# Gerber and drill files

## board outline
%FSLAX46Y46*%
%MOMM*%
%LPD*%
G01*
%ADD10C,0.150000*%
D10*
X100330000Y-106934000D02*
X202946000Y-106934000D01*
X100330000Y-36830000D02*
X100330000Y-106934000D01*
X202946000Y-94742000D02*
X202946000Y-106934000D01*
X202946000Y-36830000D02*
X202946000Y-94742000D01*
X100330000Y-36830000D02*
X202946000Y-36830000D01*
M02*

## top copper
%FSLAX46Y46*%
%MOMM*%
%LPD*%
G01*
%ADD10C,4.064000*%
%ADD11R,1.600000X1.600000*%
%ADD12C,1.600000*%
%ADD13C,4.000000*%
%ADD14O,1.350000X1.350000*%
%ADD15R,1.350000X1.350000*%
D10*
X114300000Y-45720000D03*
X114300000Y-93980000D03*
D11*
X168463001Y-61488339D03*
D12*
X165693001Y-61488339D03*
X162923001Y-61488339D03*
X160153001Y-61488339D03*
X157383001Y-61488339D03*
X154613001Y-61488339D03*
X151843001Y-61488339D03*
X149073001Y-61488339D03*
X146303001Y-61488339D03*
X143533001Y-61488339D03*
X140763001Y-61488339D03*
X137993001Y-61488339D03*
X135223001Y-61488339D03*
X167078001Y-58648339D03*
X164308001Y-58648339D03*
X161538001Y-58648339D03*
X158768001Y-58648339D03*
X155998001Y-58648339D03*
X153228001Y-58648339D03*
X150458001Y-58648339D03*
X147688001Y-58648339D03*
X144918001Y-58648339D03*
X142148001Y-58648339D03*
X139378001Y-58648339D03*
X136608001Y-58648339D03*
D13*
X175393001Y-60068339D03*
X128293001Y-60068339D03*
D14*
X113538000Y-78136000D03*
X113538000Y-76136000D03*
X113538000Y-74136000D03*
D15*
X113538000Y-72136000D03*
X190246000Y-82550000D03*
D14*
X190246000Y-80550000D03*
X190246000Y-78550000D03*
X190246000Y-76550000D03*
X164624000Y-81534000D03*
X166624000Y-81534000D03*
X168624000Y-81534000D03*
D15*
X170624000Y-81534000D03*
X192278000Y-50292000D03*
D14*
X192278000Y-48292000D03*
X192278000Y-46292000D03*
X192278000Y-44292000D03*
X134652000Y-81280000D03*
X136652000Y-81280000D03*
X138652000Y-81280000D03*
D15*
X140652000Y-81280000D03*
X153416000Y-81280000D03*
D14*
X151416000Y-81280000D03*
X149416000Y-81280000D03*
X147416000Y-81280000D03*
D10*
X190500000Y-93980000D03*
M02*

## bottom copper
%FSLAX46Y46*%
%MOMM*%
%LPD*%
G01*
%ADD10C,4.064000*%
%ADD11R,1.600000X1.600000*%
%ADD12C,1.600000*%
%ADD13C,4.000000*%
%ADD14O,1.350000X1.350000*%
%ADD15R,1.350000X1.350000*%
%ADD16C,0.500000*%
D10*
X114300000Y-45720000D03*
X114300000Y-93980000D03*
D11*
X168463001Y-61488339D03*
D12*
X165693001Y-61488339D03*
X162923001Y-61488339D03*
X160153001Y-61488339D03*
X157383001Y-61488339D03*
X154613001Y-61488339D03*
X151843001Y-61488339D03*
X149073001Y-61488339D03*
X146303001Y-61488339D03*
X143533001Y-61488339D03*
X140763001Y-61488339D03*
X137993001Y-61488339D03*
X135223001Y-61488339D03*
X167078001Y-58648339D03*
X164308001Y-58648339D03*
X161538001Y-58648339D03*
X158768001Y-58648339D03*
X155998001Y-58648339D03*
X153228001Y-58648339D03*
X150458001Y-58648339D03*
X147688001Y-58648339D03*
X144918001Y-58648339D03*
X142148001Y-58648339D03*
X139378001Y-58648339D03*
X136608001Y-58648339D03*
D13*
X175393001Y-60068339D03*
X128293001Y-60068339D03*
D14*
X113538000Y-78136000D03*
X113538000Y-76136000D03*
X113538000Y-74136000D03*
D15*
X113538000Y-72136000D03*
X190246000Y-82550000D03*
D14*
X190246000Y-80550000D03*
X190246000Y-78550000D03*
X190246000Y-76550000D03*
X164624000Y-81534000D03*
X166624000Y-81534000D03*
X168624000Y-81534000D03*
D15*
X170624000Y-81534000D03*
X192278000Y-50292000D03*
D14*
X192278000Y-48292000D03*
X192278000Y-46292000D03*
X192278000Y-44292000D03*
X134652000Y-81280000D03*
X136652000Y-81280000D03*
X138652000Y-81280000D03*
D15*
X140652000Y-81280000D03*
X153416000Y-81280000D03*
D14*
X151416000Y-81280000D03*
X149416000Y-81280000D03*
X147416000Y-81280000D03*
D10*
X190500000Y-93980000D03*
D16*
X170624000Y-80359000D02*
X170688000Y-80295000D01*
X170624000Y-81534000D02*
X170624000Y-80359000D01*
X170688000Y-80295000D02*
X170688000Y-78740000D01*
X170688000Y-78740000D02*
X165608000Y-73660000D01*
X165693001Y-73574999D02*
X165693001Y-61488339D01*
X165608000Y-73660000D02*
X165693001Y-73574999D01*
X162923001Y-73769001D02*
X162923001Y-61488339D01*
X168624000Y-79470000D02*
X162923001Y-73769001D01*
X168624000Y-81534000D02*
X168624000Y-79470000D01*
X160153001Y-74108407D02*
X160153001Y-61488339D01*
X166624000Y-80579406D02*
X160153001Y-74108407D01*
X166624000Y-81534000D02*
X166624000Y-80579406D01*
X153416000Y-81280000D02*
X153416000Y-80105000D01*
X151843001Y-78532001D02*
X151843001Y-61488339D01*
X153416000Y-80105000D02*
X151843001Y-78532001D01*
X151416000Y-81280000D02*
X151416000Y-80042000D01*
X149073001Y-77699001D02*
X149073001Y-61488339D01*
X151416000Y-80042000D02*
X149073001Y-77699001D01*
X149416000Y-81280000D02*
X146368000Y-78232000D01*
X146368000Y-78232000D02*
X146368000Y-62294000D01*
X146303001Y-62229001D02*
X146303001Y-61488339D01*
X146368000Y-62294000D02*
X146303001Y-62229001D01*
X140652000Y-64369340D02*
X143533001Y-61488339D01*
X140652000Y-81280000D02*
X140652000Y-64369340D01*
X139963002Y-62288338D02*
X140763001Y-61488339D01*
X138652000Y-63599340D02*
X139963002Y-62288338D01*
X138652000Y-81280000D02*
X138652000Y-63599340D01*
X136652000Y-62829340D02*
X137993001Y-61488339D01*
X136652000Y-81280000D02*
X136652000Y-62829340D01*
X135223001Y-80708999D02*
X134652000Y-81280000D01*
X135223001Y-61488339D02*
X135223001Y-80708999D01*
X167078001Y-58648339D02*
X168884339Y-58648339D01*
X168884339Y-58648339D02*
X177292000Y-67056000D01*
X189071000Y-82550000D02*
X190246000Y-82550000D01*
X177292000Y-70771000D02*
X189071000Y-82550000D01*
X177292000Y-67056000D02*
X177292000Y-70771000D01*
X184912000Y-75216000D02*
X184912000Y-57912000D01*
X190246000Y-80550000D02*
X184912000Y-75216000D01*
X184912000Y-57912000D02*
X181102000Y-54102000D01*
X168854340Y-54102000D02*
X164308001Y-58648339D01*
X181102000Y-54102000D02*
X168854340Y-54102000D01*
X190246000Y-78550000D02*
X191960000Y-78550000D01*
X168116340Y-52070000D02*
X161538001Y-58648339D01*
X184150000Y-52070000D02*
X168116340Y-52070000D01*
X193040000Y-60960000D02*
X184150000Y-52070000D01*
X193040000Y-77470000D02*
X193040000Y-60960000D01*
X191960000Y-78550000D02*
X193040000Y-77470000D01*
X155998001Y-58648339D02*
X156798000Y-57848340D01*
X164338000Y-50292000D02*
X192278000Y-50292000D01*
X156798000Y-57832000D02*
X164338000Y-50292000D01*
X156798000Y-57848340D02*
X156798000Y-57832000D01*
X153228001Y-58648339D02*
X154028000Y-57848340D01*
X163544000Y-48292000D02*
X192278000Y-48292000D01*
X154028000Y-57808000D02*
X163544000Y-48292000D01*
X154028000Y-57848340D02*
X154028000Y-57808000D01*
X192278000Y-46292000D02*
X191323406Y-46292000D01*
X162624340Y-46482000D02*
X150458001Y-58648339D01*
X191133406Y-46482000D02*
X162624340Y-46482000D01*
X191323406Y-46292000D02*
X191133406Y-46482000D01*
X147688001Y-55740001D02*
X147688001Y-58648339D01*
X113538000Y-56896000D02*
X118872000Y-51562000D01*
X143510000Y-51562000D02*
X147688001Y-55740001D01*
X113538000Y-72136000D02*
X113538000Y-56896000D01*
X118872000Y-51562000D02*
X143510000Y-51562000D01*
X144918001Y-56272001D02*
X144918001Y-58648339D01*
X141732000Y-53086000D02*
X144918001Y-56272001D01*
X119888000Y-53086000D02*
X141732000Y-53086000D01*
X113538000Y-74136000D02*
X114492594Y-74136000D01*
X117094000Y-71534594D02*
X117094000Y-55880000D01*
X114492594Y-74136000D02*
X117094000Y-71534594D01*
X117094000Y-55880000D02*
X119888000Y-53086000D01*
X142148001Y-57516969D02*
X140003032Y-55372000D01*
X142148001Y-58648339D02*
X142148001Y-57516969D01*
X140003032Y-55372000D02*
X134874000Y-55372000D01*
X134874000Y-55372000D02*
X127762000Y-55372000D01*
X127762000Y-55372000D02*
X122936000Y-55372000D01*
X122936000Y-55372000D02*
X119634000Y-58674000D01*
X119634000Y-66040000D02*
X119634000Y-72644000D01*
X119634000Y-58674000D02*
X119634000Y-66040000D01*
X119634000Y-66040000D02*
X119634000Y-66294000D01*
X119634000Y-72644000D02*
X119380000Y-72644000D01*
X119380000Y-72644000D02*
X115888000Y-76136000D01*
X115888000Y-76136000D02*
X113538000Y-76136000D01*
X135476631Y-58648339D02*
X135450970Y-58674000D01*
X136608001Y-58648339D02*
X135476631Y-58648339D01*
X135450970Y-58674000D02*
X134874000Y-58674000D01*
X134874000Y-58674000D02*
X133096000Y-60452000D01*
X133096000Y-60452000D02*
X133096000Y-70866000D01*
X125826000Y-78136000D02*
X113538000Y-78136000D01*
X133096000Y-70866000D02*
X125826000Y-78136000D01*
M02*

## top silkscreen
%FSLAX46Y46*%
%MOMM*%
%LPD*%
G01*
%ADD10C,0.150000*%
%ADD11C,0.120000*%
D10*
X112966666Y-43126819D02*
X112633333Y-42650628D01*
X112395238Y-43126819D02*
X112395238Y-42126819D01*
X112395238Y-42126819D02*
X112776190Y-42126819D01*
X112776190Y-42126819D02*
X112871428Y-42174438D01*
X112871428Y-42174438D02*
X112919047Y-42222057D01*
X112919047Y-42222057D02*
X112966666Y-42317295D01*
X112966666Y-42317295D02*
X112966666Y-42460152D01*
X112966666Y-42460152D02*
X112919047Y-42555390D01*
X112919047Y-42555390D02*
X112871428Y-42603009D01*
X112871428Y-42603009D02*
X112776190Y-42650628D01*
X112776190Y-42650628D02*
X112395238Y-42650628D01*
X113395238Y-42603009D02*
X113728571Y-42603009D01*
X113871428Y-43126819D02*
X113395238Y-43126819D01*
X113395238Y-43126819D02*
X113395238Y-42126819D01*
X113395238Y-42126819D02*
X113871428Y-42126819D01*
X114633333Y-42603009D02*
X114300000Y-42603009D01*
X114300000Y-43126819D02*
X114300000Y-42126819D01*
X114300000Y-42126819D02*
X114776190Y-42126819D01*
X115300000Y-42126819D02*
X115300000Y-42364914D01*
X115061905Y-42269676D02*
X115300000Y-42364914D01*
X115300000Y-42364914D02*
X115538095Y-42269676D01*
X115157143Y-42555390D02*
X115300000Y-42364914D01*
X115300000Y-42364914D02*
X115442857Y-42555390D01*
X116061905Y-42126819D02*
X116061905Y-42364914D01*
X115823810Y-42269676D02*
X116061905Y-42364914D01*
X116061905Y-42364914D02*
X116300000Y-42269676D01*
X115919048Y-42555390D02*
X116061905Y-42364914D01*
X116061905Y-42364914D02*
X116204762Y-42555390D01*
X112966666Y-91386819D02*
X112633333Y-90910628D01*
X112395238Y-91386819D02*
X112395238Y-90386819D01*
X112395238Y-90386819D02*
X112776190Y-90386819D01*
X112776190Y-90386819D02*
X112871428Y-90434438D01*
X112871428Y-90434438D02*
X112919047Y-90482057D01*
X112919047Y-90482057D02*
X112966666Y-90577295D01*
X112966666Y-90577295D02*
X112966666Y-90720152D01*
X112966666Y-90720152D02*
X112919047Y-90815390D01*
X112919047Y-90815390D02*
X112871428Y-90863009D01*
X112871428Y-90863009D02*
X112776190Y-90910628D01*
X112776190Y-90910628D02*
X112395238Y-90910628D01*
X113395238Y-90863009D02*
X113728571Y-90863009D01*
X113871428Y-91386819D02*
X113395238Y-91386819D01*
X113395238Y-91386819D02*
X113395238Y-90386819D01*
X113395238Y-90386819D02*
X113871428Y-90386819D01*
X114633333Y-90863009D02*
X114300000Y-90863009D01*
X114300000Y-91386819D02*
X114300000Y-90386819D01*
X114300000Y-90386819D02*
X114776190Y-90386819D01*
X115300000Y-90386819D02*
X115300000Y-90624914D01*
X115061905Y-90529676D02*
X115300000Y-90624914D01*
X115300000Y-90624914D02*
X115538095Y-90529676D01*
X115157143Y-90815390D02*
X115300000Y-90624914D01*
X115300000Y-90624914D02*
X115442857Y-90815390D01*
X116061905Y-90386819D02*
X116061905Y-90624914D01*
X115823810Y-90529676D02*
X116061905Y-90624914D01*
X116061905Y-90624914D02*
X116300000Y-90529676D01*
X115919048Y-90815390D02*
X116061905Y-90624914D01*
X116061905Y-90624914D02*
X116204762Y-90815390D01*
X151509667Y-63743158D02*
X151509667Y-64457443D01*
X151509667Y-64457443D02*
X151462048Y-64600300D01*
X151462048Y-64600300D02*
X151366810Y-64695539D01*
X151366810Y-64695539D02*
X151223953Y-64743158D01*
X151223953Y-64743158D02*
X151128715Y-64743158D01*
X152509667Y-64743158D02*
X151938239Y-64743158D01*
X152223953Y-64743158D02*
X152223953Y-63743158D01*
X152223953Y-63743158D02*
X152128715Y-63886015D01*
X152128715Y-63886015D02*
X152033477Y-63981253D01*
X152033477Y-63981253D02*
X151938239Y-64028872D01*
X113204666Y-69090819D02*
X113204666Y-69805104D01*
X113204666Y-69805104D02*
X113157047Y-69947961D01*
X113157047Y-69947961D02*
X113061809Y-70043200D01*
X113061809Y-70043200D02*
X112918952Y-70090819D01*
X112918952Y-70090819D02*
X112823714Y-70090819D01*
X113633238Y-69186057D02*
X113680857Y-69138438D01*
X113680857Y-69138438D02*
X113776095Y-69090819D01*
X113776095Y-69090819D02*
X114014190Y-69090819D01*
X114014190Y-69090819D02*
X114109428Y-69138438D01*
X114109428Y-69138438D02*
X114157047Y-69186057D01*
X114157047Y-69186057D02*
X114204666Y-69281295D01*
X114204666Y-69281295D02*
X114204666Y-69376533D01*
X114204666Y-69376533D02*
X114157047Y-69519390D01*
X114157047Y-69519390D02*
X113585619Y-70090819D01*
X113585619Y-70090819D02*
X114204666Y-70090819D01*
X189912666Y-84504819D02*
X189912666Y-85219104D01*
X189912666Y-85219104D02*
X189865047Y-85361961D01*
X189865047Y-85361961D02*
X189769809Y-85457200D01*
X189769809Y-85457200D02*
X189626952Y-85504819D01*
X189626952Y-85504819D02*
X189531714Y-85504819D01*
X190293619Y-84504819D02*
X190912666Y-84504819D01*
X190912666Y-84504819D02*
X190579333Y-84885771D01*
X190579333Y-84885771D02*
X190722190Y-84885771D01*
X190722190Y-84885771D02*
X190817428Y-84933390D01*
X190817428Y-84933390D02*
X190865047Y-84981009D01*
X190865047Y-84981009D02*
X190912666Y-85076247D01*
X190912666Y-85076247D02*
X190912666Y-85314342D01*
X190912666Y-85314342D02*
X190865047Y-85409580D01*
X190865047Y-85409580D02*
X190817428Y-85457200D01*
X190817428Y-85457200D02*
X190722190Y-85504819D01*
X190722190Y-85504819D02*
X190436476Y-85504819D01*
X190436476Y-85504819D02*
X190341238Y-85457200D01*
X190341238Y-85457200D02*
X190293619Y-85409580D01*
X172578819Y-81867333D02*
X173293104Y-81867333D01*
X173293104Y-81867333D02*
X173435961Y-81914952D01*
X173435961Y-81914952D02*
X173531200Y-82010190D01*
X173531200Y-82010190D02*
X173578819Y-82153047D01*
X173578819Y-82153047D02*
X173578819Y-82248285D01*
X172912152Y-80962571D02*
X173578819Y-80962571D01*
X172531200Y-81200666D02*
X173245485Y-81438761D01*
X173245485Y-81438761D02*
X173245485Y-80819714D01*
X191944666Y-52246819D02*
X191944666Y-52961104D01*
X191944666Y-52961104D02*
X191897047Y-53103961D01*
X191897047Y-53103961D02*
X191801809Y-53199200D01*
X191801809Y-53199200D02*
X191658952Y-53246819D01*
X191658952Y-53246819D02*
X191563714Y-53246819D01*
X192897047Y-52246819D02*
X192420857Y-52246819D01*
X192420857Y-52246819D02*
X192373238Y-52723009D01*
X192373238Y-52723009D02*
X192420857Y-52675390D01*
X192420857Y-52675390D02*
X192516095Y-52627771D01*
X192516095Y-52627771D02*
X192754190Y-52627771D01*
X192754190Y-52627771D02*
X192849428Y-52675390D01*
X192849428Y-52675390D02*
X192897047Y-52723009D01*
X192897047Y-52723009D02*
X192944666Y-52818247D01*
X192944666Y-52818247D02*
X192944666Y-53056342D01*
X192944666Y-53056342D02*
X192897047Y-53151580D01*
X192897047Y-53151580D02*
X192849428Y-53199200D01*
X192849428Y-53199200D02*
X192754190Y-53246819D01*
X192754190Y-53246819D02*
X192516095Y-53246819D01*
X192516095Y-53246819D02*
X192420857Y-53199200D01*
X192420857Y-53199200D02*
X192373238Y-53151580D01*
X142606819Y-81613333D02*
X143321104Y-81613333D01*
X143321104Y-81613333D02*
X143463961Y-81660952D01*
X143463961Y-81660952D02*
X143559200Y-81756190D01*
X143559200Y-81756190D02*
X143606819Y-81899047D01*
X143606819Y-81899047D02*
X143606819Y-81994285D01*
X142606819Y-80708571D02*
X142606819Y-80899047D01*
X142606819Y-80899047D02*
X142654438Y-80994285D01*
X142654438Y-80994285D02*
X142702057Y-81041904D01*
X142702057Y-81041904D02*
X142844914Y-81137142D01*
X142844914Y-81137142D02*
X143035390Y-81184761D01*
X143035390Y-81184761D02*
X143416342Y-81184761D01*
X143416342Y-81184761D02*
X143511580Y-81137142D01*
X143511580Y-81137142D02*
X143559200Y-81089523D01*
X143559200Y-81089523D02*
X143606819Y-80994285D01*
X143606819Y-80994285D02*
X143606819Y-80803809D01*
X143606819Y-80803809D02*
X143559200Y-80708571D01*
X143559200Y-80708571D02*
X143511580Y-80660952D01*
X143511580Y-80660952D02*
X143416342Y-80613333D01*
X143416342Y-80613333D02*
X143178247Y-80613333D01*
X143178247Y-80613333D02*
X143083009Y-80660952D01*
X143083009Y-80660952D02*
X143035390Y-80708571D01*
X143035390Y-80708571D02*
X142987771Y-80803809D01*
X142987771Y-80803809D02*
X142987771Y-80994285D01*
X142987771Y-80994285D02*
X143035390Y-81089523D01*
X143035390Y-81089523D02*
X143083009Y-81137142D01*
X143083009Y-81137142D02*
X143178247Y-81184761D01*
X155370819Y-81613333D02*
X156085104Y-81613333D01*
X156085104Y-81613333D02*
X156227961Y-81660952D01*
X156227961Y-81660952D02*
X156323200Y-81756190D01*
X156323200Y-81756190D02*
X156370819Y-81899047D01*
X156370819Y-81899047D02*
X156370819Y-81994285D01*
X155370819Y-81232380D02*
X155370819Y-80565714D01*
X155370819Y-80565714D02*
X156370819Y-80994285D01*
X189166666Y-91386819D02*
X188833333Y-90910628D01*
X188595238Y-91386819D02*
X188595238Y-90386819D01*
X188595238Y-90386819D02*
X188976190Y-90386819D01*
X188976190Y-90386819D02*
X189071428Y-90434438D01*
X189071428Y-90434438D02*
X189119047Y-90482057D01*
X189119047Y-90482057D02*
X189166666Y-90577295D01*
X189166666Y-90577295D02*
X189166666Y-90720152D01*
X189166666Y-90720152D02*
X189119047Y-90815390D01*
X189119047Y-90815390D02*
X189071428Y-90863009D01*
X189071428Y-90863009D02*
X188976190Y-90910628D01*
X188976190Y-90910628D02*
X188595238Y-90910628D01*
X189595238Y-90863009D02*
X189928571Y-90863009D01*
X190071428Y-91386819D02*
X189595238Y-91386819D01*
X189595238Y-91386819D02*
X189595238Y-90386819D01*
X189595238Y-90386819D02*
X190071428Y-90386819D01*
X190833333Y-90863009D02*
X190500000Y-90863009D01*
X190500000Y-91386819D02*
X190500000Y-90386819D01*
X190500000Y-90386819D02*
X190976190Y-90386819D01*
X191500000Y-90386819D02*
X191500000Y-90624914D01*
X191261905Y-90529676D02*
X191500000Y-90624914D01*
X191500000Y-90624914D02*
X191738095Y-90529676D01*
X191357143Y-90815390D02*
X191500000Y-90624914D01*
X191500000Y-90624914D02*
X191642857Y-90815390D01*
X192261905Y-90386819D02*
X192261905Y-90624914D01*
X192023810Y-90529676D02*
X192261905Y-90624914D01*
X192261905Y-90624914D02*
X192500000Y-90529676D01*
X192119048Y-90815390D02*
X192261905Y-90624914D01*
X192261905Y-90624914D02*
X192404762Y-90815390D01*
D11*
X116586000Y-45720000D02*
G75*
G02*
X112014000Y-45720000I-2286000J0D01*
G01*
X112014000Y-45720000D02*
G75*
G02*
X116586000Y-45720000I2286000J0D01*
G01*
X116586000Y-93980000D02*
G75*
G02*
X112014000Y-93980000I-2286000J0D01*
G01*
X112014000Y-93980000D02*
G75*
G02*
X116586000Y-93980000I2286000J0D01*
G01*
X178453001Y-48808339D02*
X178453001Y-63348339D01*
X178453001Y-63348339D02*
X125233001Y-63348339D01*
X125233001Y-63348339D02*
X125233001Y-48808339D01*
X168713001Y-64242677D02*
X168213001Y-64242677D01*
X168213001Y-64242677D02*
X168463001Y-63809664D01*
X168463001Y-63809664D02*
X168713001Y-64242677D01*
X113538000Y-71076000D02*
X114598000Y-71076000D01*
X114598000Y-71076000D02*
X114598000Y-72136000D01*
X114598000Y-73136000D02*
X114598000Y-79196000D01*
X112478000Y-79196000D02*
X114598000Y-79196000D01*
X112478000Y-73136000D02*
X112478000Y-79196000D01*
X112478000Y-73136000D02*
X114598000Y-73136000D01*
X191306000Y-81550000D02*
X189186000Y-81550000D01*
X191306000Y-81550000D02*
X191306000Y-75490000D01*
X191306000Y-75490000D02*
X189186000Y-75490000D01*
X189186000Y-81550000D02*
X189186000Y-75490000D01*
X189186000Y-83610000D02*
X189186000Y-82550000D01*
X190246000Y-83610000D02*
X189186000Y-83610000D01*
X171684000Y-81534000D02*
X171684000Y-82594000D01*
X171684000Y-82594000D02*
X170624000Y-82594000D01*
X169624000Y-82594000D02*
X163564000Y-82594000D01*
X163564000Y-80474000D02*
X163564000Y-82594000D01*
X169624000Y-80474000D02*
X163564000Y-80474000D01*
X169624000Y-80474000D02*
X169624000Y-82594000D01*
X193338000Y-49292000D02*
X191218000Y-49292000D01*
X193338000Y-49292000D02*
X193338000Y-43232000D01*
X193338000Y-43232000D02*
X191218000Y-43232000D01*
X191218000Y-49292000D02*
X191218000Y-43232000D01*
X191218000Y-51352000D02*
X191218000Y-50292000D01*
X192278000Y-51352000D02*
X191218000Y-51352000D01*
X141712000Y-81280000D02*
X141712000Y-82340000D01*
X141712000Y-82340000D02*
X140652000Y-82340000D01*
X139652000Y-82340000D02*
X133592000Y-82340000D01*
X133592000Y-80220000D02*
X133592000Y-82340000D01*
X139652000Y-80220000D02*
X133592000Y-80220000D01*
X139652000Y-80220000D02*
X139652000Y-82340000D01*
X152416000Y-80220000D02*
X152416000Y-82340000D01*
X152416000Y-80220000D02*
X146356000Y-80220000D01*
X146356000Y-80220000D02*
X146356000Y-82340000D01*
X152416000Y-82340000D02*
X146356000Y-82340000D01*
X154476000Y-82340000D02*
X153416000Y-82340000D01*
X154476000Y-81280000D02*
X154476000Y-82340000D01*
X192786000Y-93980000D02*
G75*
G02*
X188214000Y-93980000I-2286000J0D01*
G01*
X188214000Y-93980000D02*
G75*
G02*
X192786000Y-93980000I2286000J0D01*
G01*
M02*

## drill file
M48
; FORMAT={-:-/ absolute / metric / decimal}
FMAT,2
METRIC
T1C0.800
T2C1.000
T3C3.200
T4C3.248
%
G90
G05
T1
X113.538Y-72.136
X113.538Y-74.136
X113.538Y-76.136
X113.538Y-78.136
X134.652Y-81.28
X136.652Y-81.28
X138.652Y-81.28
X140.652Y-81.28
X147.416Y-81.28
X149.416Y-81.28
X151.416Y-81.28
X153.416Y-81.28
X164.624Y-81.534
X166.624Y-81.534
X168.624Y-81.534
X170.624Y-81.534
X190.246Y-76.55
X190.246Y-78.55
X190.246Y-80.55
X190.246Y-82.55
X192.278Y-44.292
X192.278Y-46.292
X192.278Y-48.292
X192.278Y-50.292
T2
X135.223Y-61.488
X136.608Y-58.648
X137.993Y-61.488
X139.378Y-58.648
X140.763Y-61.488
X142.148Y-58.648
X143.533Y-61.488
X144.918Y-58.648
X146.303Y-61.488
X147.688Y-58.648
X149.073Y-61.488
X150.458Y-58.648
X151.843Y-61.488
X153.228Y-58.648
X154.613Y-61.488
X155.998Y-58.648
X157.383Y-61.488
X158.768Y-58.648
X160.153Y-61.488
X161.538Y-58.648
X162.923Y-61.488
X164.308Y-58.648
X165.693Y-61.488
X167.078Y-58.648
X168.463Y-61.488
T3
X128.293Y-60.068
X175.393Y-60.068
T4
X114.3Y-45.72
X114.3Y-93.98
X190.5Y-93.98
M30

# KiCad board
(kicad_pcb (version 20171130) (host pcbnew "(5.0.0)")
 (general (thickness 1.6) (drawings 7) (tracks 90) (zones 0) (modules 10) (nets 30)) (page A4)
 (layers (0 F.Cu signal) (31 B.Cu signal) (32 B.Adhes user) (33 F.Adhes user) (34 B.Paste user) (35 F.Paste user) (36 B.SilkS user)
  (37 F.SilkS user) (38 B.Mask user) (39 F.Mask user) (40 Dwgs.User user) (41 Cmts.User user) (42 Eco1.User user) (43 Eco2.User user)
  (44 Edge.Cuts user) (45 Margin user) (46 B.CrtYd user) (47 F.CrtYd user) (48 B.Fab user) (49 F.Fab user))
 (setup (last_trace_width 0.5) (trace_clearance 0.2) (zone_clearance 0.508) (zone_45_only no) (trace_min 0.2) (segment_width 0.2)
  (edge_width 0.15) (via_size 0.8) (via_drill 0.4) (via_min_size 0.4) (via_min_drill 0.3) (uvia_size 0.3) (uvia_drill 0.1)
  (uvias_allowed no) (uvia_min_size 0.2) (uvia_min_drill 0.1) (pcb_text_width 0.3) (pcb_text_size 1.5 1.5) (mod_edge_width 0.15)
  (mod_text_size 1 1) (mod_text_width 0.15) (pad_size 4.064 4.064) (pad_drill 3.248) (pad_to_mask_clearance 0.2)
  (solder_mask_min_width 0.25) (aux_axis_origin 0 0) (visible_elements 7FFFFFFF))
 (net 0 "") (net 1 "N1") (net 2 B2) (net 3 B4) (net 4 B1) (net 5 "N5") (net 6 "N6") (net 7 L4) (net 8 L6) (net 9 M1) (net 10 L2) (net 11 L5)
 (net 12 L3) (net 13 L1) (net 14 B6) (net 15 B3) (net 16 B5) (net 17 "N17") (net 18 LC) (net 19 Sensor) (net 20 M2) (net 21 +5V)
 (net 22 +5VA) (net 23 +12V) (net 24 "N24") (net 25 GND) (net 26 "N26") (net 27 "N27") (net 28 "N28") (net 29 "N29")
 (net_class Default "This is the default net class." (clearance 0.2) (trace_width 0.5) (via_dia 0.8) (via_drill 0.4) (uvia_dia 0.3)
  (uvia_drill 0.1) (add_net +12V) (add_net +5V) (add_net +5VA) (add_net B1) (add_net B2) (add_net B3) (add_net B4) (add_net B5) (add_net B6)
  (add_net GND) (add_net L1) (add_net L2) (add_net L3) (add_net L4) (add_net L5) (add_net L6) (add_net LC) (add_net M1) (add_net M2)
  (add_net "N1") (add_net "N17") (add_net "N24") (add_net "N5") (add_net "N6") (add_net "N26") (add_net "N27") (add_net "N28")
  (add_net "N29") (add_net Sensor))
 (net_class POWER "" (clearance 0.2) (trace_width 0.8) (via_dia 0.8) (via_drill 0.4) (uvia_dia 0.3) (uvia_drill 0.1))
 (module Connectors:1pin (layer F.Cu) (at 114.3 45.72)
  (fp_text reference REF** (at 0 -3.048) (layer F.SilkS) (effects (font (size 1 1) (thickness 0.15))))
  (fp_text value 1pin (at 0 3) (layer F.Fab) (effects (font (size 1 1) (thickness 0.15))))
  (fp_circle (center 0 0) (end 0 -2.286) (layer F.SilkS) (width 0.12))
  (pad 1 thru_hole circle (at 0 0) (size 4.064 4.064) (drill 3.248) (layers *.Cu *.Mask)))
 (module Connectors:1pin (layer F.Cu) (at 114.3 93.98)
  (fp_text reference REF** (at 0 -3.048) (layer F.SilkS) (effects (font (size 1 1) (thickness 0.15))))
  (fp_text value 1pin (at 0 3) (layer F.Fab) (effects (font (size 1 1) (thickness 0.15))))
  (fp_circle (center 0 0) (end 0 -2.286) (layer F.SilkS) (width 0.12))
  (pad 1 thru_hole circle (at 0 0) (size 4.064 4.064) (drill 3.248) (layers *.Cu *.Mask)))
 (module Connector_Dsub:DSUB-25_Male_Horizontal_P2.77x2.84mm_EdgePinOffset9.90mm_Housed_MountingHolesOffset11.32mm (layer F.Cu)
  (at 168.463001 61.488339 180)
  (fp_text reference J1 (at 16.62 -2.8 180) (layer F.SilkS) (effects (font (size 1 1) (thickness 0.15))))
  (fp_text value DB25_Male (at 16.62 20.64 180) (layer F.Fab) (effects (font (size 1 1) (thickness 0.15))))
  (fp_line (start -9.99 12.68) (end -9.99 -1.86) (layer F.SilkS) (width 0.12))
  (fp_line (start -9.99 -1.86) (end 43.23 -1.86) (layer F.SilkS) (width 0.12))
  (fp_line (start 43.23 -1.86) (end 43.23 12.68) (layer F.SilkS) (width 0.12))
  (fp_line (start -0.25 -2.754338) (end 0.25 -2.754338) (layer F.SilkS) (width 0.12))
  (fp_line (start 0.25 -2.754338) (end 0 -2.321325) (layer F.SilkS) (width 0.12))
  (fp_line (start 0 -2.321325) (end -0.25 -2.754338) (layer F.SilkS) (width 0.12))
  (pad 1 thru_hole rect (at 0 0 180) (size 1.6 1.6) (drill 1) (layers *.Cu *.Mask) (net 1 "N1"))
  (pad 2 thru_hole circle (at 2.77 0 180) (size 1.6 1.6) (drill 1) (layers *.Cu *.Mask) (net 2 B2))
  (pad 3 thru_hole circle (at 5.54 0 180) (size 1.6 1.6) (drill 1) (layers *.Cu *.Mask) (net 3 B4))
  (pad 4 thru_hole circle (at 8.31 0 180) (size 1.6 1.6) (drill 1) (layers *.Cu *.Mask) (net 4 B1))
  (pad 5 thru_hole circle (at 11.08 0 180) (size 1.6 1.6) (drill 1) (layers *.Cu *.Mask) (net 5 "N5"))
  (pad 6 thru_hole circle (at 13.85 0 180) (size 1.6 1.6) (drill 1) (layers *.Cu *.Mask) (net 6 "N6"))
  (pad 7 thru_hole circle (at 16.62 0 180) (size 1.6 1.6) (drill 1) (layers *.Cu *.Mask) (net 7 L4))
  (pad 8 thru_hole circle (at 19.39 0 180) (size 1.6 1.6) (drill 1) (layers *.Cu *.Mask) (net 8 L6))
  (pad 9 thru_hole circle (at 22.16 0 180) (size 1.6 1.6) (drill 1) (layers *.Cu *.Mask) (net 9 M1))
  (pad 10 thru_hole circle (at 24.93 0 180) (size 1.6 1.6) (drill 1) (layers *.Cu *.Mask) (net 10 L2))
  (pad 11 thru_hole circle (at 27.7 0 180) (size 1.6 1.6) (drill 1) (layers *.Cu *.Mask) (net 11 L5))
  (pad 12 thru_hole circle (at 30.47 0 180) (size 1.6 1.6) (drill 1) (layers *.Cu *.Mask) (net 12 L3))
  (pad 13 thru_hole circle (at 33.24 0 180) (size 1.6 1.6) (drill 1) (layers *.Cu *.Mask) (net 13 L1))
  (pad 14 thru_hole circle (at 1.385 2.84 180) (size 1.6 1.6) (drill 1) (layers *.Cu *.Mask) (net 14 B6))
  (pad 15 thru_hole circle (at 4.155 2.84 180) (size 1.6 1.6) (drill 1) (layers *.Cu *.Mask) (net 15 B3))
  (pad 16 thru_hole circle (at 6.925 2.84 180) (size 1.6 1.6) (drill 1) (layers *.Cu *.Mask) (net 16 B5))
  (pad 17 thru_hole circle (at 9.695 2.84 180) (size 1.6 1.6) (drill 1) (layers *.Cu *.Mask) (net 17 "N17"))
  (pad 18 thru_hole circle (at 12.465 2.84 180) (size 1.6 1.6) (drill 1) (layers *.Cu *.Mask) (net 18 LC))
  (pad 19 thru_hole circle (at 15.235 2.84 180) (size 1.6 1.6) (drill 1) (layers *.Cu *.Mask) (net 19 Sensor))
  (pad 20 thru_hole circle (at 18.005 2.84 180) (size 1.6 1.6) (drill 1) (layers *.Cu *.Mask) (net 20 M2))
  (pad 21 thru_hole circle (at 20.775 2.84 180) (size 1.6 1.6) (drill 1) (layers *.Cu *.Mask) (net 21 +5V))
  (pad 22 thru_hole circle (at 23.545 2.84 180) (size 1.6 1.6) (drill 1) (layers *.Cu *.Mask) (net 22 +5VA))
  (pad 23 thru_hole circle (at 26.315 2.84 180) (size 1.6 1.6) (drill 1) (layers *.Cu *.Mask) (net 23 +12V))
  (pad 24 thru_hole circle (at 29.085 2.84 180) (size 1.6 1.6) (drill 1) (layers *.Cu *.Mask) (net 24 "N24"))
  (pad 25 thru_hole circle (at 31.855 2.84 180) (size 1.6 1.6) (drill 1) (layers *.Cu *.Mask) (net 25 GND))
  (pad 0 thru_hole circle (at -6.93 1.42 180) (size 4 4) (drill 3.2) (layers *.Cu *.Mask))
  (pad 0 thru_hole circle (at 40.17 1.42 180) (size 4 4) (drill 3.2) (layers *.Cu *.Mask)))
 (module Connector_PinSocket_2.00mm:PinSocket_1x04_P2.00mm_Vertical (layer F.Cu) (at 113.538 72.136)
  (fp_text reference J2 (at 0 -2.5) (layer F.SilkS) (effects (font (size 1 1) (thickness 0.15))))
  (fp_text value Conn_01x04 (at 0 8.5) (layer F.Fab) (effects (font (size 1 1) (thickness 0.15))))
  (fp_line (start 0 -1.06) (end 1.06 -1.06) (layer F.SilkS) (width 0.12))
  (fp_line (start 1.06 -1.06) (end 1.06 0) (layer F.SilkS) (width 0.12))
  (fp_line (start 1.06 1) (end 1.06 7.06) (layer F.SilkS) (width 0.12))
  (fp_line (start -1.06 7.06) (end 1.06 7.06) (layer F.SilkS) (width 0.12))
  (fp_line (start -1.06 1) (end -1.06 7.06) (layer F.SilkS) (width 0.12))
  (fp_line (start -1.06 1) (end 1.06 1) (layer F.SilkS) (width 0.12))
  (pad 4 thru_hole oval (at 0 6) (size 1.35 1.35) (drill 0.8) (layers *.Cu *.Mask) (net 25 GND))
  (pad 3 thru_hole oval (at 0 4) (size 1.35 1.35) (drill 0.8) (layers *.Cu *.Mask) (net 23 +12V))
  (pad 2 thru_hole oval (at 0 2) (size 1.35 1.35) (drill 0.8) (layers *.Cu *.Mask) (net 22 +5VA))
  (pad 1 thru_hole rect (at 0 0) (size 1.35 1.35) (drill 0.8) (layers *.Cu *.Mask) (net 21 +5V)))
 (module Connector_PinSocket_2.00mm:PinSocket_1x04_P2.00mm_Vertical (layer F.Cu) (at 190.246 82.55 180)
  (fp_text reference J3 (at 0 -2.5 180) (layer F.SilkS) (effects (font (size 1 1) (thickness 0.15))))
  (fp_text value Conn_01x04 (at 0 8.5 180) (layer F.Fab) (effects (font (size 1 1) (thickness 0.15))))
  (fp_line (start -1.06 1) (end 1.06 1) (layer F.SilkS) (width 0.12))
  (fp_line (start -1.06 1) (end -1.06 7.06) (layer F.SilkS) (width 0.12))
  (fp_line (start -1.06 7.06) (end 1.06 7.06) (layer F.SilkS) (width 0.12))
  (fp_line (start 1.06 1) (end 1.06 7.06) (layer F.SilkS) (width 0.12))
  (fp_line (start 1.06 -1.06) (end 1.06 0) (layer F.SilkS) (width 0.12))
  (fp_line (start 0 -1.06) (end 1.06 -1.06) (layer F.SilkS) (width 0.12))
  (pad 1 thru_hole rect (at 0 0 180) (size 1.35 1.35) (drill 0.8) (layers *.Cu *.Mask) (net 14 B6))
  (pad 2 thru_hole oval (at 0 2 180) (size 1.35 1.35) (drill 0.8) (layers *.Cu *.Mask) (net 15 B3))
  (pad 3 thru_hole oval (at 0 4 180) (size 1.35 1.35) (drill 0.8) (layers *.Cu *.Mask) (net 16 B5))
  (pad 4 thru_hole oval (at 0 6 180) (size 1.35 1.35) (drill 0.8) (layers *.Cu *.Mask) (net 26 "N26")))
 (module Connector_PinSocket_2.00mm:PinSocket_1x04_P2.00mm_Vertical (layer F.Cu) (at 170.624 81.534 270)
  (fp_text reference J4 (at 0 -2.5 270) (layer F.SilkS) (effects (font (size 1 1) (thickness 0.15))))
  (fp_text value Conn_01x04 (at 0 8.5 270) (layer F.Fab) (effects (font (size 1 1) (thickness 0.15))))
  (fp_line (start 0 -1.06) (end 1.06 -1.06) (layer F.SilkS) (width 0.12))
  (fp_line (start 1.06 -1.06) (end 1.06 0) (layer F.SilkS) (width 0.12))
  (fp_line (start 1.06 1) (end 1.06 7.06) (layer F.SilkS) (width 0.12))
  (fp_line (start -1.06 7.06) (end 1.06 7.06) (layer F.SilkS) (width 0.12))
  (fp_line (start -1.06 1) (end -1.06 7.06) (layer F.SilkS) (width 0.12))
  (fp_line (start -1.06 1) (end 1.06 1) (layer F.SilkS) (width 0.12))
  (pad 4 thru_hole oval (at 0 6 270) (size 1.35 1.35) (drill 0.8) (layers *.Cu *.Mask) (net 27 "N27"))
  (pad 3 thru_hole oval (at 0 4 270) (size 1.35 1.35) (drill 0.8) (layers *.Cu *.Mask) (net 4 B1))
  (pad 2 thru_hole oval (at 0 2 270) (size 1.35 1.35) (drill 0.8) (layers *.Cu *.Mask) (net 3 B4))
  (pad 1 thru_hole rect (at 0 0 270) (size 1.35 1.35) (drill 0.8) (layers *.Cu *.Mask) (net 2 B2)))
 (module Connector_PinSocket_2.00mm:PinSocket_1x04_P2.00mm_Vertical (layer F.Cu) (at 192.278 50.292 180)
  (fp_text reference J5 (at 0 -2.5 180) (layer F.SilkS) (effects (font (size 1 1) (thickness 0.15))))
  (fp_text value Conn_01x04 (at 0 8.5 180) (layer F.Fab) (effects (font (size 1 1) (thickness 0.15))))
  (fp_line (start -1.06 1) (end 1.06 1) (layer F.SilkS) (width 0.12))
  (fp_line (start -1.06 1) (end -1.06 7.06) (layer F.SilkS) (width 0.12))
  (fp_line (start -1.06 7.06) (end 1.06 7.06) (layer F.SilkS) (width 0.12))
  (fp_line (start 1.06 1) (end 1.06 7.06) (layer F.SilkS) (width 0.12))
  (fp_line (start 1.06 -1.06) (end 1.06 0) (layer F.SilkS) (width 0.12))
  (fp_line (start 0 -1.06) (end 1.06 -1.06) (layer F.SilkS) (width 0.12))
  (pad 1 thru_hole rect (at 0 0 180) (size 1.35 1.35) (drill 0.8) (layers *.Cu *.Mask) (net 18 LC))
  (pad 2 thru_hole oval (at 0 2 180) (size 1.35 1.35) (drill 0.8) (layers *.Cu *.Mask) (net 19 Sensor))
  (pad 3 thru_hole oval (at 0 4 180) (size 1.35 1.35) (drill 0.8) (layers *.Cu *.Mask) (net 20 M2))
  (pad 4 thru_hole oval (at 0 6 180) (size 1.35 1.35) (drill 0.8) (layers *.Cu *.Mask) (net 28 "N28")))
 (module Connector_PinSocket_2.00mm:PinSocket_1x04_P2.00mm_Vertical (layer F.Cu) (at 140.652 81.28 270)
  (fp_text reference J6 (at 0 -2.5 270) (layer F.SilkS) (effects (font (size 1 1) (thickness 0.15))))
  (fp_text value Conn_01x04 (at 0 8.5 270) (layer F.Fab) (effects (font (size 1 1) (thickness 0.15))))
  (fp_line (start 0 -1.06) (end 1.06 -1.06) (layer F.SilkS) (width 0.12))
  (fp_line (start 1.06 -1.06) (end 1.06 0) (layer F.SilkS) (width 0.12))
  (fp_line (start 1.06 1) (end 1.06 7.06) (layer F.SilkS) (width 0.12))
  (fp_line (start -1.06 7.06) (end 1.06 7.06) (layer F.SilkS) (width 0.12))
  (fp_line (start -1.06 1) (end -1.06 7.06) (layer F.SilkS) (width 0.12))
  (fp_line (start -1.06 1) (end 1.06 1) (layer F.SilkS) (width 0.12))
  (pad 4 thru_hole oval (at 0 6 270) (size 1.35 1.35) (drill 0.8) (layers *.Cu *.Mask) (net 13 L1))
  (pad 3 thru_hole oval (at 0 4 270) (size 1.35 1.35) (drill 0.8) (layers *.Cu *.Mask) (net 12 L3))
  (pad 2 thru_hole oval (at 0 2 270) (size 1.35 1.35) (drill 0.8) (layers *.Cu *.Mask) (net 11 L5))
  (pad 1 thru_hole rect (at 0 0 270) (size 1.35 1.35) (drill 0.8) (layers *.Cu *.Mask) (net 10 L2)))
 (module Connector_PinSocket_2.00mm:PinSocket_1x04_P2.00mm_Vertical (layer F.Cu) (at 153.416 81.28 270)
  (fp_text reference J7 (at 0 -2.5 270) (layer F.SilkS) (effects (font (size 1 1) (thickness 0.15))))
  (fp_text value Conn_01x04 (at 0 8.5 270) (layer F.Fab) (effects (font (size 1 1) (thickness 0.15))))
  (fp_line (start -1.06 1) (end 1.06 1) (layer F.SilkS) (width 0.12))
  (fp_line (start -1.06 1) (end -1.06 7.06) (layer F.SilkS) (width 0.12))
  (fp_line (start -1.06 7.06) (end 1.06 7.06) (layer F.SilkS) (width 0.12))
  (fp_line (start 1.06 1) (end 1.06 7.06) (layer F.SilkS) (width 0.12))
  (fp_line (start 1.06 -1.06) (end 1.06 0) (layer F.SilkS) (width 0.12))
  (fp_line (start 0 -1.06) (end 1.06 -1.06) (layer F.SilkS) (width 0.12))
  (pad 1 thru_hole rect (at 0 0 270) (size 1.35 1.35) (drill 0.8) (layers *.Cu *.Mask) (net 7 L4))
  (pad 2 thru_hole oval (at 0 2 270) (size 1.35 1.35) (drill 0.8) (layers *.Cu *.Mask) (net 8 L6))
  (pad 3 thru_hole oval (at 0 4 270) (size 1.35 1.35) (drill 0.8) (layers *.Cu *.Mask) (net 9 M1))
  (pad 4 thru_hole oval (at 0 6 270) (size 1.35 1.35) (drill 0.8) (layers *.Cu *.Mask) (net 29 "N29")))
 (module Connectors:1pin (layer F.Cu) (at 190.5 93.98)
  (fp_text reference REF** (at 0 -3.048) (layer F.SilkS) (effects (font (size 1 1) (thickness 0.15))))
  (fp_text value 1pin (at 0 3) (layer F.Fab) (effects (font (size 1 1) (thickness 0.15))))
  (fp_circle (center 0 0) (end 0 -2.286) (layer F.SilkS) (width 0.12))
  (pad 1 thru_hole circle (at 0 0) (size 4.064 4.064) (drill 3.248) (layers *.Cu *.Mask)))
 (gr_line (start 100.33 106.934) (end 202.946 106.934) (layer Edge.Cuts) (width 0.15))
 (gr_line (start 100.33 36.83) (end 100.33 106.934) (layer Edge.Cuts) (width 0.15))
 (gr_line (start 202.946 94.742) (end 202.946 106.934) (layer Edge.Cuts) (width 0.15))
 (gr_line (start 202.946 36.83) (end 202.946 94.742) (layer Edge.Cuts) (width 0.15))
 (gr_line (start 100.33 36.83) (end 202.946 36.83) (layer Edge.Cuts) (width 0.15))
 (segment (start 170.624 80.359) (end 170.688 80.295) (width 0.5) (layer B.Cu) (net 2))
 (segment (start 170.624 81.534) (end 170.624 80.359) (width 0.5) (layer B.Cu) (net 2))
 (segment (start 170.688 80.295) (end 170.688 78.74) (width 0.5) (layer B.Cu) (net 2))
 (segment (start 170.688 78.74) (end 165.608 73.66) (width 0.5) (layer B.Cu) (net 2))
 (segment (start 165.693001 73.574999) (end 165.693001 61.488339) (width 0.5) (layer B.Cu) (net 2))
 (segment (start 165.608 73.66) (end 165.693001 73.574999) (width 0.5) (layer B.Cu) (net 2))
 (segment (start 162.923001 73.769001) (end 162.923001 61.488339) (width 0.5) (layer B.Cu) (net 3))
 (segment (start 168.624 79.47) (end 162.923001 73.769001) (width 0.5) (layer B.Cu) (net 3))
 (segment (start 168.624 81.534) (end 168.624 79.47) (width 0.5) (layer B.Cu) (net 3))
 (segment (start 160.153001 74.108407) (end 160.153001 61.488339) (width 0.5) (layer B.Cu) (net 4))
 (segment (start 166.624 80.579406) (end 160.153001 74.108407) (width 0.5) (layer B.Cu) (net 4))
 (segment (start 166.624 81.534) (end 166.624 80.579406) (width 0.5) (layer B.Cu) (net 4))
 (segment (start 153.416 81.28) (end 153.416 80.105) (width 0.5) (layer B.Cu) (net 7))
 (segment (start 151.843001 78.532001) (end 151.843001 61.488339) (width 0.5) (layer B.Cu) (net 7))
 (segment (start 153.416 80.105) (end 151.843001 78.532001) (width 0.5) (layer B.Cu) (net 7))
 (segment (start 151.416 81.28) (end 151.416 80.042) (width 0.5) (layer B.Cu) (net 8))
 (segment (start 149.073001 77.699001) (end 149.073001 61.488339) (width 0.5) (layer B.Cu) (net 8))
 (segment (start 151.416 80.042) (end 149.073001 77.699001) (width 0.5) (layer B.Cu) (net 8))
 (segment (start 149.416 81.28) (end 146.368 78.232) (width 0.5) (layer B.Cu) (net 9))
 (segment (start 146.368 78.232) (end 146.368 62.294) (width 0.5) (layer B.Cu) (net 9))
 (segment (start 146.303001 62.229001) (end 146.303001 61.488339) (width 0.5) (layer B.Cu) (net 9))
 (segment (start 146.368 62.294) (end 146.303001 62.229001) (width 0.5) (layer B.Cu) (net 9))
 (segment (start 140.652 64.36934) (end 143.533001 61.488339) (width 0.5) (layer B.Cu) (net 10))
 (segment (start 140.652 81.28) (end 140.652 64.36934) (width 0.5) (layer B.Cu) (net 10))
 (segment (start 139.963002 62.288338) (end 140.763001 61.488339) (width 0.5) (layer B.Cu) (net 11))
 (segment (start 138.652 63.59934) (end 139.963002 62.288338) (width 0.5) (layer B.Cu) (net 11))
 (segment (start 138.652 81.28) (end 138.652 63.59934) (width 0.5) (layer B.Cu) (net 11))
 (segment (start 136.652 62.82934) (end 137.993001 61.488339) (width 0.5) (layer B.Cu) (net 12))
 (segment (start 136.652 81.28) (end 136.652 62.82934) (width 0.5) (layer B.Cu) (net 12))
 (segment (start 135.223001 80.708999) (end 134.652 81.28) (width 0.5) (layer B.Cu) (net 13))
 (segment (start 135.223001 61.488339) (end 135.223001 80.708999) (width 0.5) (layer B.Cu) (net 13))
 (segment (start 167.078001 58.648339) (end 168.884339 58.648339) (width 0.5) (layer B.Cu) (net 14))
 (segment (start 168.884339 58.648339) (end 177.292 67.056) (width 0.5) (layer B.Cu) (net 14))
 (segment (start 189.071 82.55) (end 190.246 82.55) (width 0.5) (layer B.Cu) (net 14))
 (segment (start 177.292 70.771) (end 189.071 82.55) (width 0.5) (layer B.Cu) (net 14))
 (segment (start 177.292 67.056) (end 177.292 70.771) (width 0.5) (layer B.Cu) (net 14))
 (segment (start 184.912 75.216) (end 184.912 57.912) (width 0.5) (layer B.Cu) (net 15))
 (segment (start 190.246 80.55) (end 184.912 75.216) (width 0.5) (layer B.Cu) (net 15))
 (segment (start 184.912 57.912) (end 181.102 54.102) (width 0.5) (layer B.Cu) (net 15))
 (segment (start 168.85434 54.102) (end 164.308001 58.648339) (width 0.5) (layer B.Cu) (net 15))
 (segment (start 181.102 54.102) (end 168.85434 54.102) (width 0.5) (layer B.Cu) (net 15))
 (segment (start 190.246 78.55) (end 191.96 78.55) (width 0.5) (layer B.Cu) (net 16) (status 400000))
 (segment (start 168.11634 52.07) (end 161.538001 58.648339) (width 0.5) (layer B.Cu) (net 16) (status 800000))
 (segment (start 184.15 52.07) (end 168.11634 52.07) (width 0.5) (layer B.Cu) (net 16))
 (segment (start 193.04 60.96) (end 184.15 52.07) (width 0.5) (layer B.Cu) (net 16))
 (segment (start 193.04 77.47) (end 193.04 60.96) (width 0.5) (layer B.Cu) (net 16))
 (segment (start 191.96 78.55) (end 193.04 77.47) (width 0.5) (layer B.Cu) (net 16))
 (segment (start 155.998001 58.648339) (end 156.798 57.84834) (width 0.5) (layer B.Cu) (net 18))
 (segment (start 164.338 50.292) (end 192.278 50.292) (width 0.5) (layer B.Cu) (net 18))
 (segment (start 156.798 57.832) (end 164.338 50.292) (width 0.5) (layer B.Cu) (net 18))
 (segment (start 156.798 57.84834) (end 156.798 57.832) (width 0.5) (layer B.Cu) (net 18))
 (segment (start 153.228001 58.648339) (end 154.028 57.84834) (width 0.5) (layer B.Cu) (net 19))
 (segment (start 163.544 48.292) (end 192.278 48.292) (width 0.5) (layer B.Cu) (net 19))
 (segment (start 154.028 57.808) (end 163.544 48.292) (width 0.5) (layer B.Cu) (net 19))
 (segment (start 154.028 57.84834) (end 154.028 57.808) (width 0.5) (layer B.Cu) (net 19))
 (segment (start 192.278 46.292) (end 191.323406 46.292) (width 0.5) (layer B.Cu) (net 20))
 (segment (start 162.62434 46.482) (end 150.458001 58.648339) (width 0.5) (layer B.Cu) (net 20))
 (segment (start 191.133406 46.482) (end 162.62434 46.482) (width 0.5) (layer B.Cu) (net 20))
 (segment (start 191.323406 46.292) (end 191.133406 46.482) (width 0.5) (layer B.Cu) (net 20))
 (segment (start 147.688001 55.740001) (end 147.688001 58.648339) (width 0.5) (layer B.Cu) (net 21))
 (segment (start 113.538 56.896) (end 118.872 51.562) (width 0.5) (layer B.Cu) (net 21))
 (segment (start 143.51 51.562) (end 147.688001 55.740001) (width 0.5) (layer B.Cu) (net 21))
 (segment (start 113.538 72.136) (end 113.538 56.896) (width 0.5) (layer B.Cu) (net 21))
 (segment (start 118.872 51.562) (end 143.51 51.562) (width 0.5) (layer B.Cu) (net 21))
 (segment (start 144.918001 56.272001) (end 144.918001 58.648339) (width 0.5) (layer B.Cu) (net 22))
 (segment (start 141.732 53.086) (end 144.918001 56.272001) (width 0.5) (layer B.Cu) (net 22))
 (segment (start 119.888 53.086) (end 141.732 53.086) (width 0.5) (layer B.Cu) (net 22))
 (segment (start 113.538 74.136) (end 114.492594 74.136) (width 0.5) (layer B.Cu) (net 22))
 (segment (start 117.094 71.534594) (end 117.094 55.88) (width 0.5) (layer B.Cu) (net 22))
 (segment (start 114.492594 74.136) (end 117.094 71.534594) (width 0.5) (layer B.Cu) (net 22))
 (segment (start 117.094 55.88) (end 119.888 53.086) (width 0.5) (layer B.Cu) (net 22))
 (segment (start 142.148001 57.516969) (end 140.003032 55.372) (width 0.5) (layer B.Cu) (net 23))
 (segment (start 142.148001 58.648339) (end 142.148001 57.516969) (width 0.5) (layer B.Cu) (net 23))
 (segment (start 140.003032 55.372) (end 134.874 55.372) (width 0.5) (layer B.Cu) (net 23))
 (segment (start 134.874 55.372) (end 127.762 55.372) (width 0.5) (layer B.Cu) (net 23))
 (segment (start 127.762 55.372) (end 122.936 55.372) (width 0.5) (layer B.Cu) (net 23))
 (segment (start 122.936 55.372) (end 119.634 58.674) (width 0.5) (layer B.Cu) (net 23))
 (segment (start 119.634 66.04) (end 119.634 72.644) (width 0.5) (layer B.Cu) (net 23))
 (segment (start 119.634 58.674) (end 119.634 66.04) (width 0.5) (layer B.Cu) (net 23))
 (segment (start 119.634 66.04) (end 119.634 66.294) (width 0.5) (layer B.Cu) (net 23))
 (segment (start 119.634 72.644) (end 119.38 72.644) (width 0.5) (layer B.Cu) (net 23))
 (segment (start 119.38 72.644) (end 115.888 76.136) (width 0.5) (layer B.Cu) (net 23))
 (segment (start 115.888 76.136) (end 113.538 76.136) (width 0.5) (layer B.Cu) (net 23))
 (segment (start 135.476631 58.648339) (end 135.45097 58.674) (width 0.5) (layer B.Cu) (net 25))
 (segment (start 136.608001 58.648339) (end 135.476631 58.648339) (width 0.5) (layer B.Cu) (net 25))
 (segment (start 135.45097 58.674) (end 134.874 58.674) (width 0.5) (layer B.Cu) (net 25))
 (segment (start 134.874 58.674) (end 133.096 60.452) (width 0.5) (layer B.Cu) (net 25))
 (segment (start 133.096 60.452) (end 133.096 70.866) (width 0.5) (layer B.Cu) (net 25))
 (segment (start 125.826 78.136) (end 113.538 78.136) (width 0.5) (layer B.Cu) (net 25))
 (segment (start 133.096 70.866) (end 125.826 78.136) (width 0.5) (layer B.Cu) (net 25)))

